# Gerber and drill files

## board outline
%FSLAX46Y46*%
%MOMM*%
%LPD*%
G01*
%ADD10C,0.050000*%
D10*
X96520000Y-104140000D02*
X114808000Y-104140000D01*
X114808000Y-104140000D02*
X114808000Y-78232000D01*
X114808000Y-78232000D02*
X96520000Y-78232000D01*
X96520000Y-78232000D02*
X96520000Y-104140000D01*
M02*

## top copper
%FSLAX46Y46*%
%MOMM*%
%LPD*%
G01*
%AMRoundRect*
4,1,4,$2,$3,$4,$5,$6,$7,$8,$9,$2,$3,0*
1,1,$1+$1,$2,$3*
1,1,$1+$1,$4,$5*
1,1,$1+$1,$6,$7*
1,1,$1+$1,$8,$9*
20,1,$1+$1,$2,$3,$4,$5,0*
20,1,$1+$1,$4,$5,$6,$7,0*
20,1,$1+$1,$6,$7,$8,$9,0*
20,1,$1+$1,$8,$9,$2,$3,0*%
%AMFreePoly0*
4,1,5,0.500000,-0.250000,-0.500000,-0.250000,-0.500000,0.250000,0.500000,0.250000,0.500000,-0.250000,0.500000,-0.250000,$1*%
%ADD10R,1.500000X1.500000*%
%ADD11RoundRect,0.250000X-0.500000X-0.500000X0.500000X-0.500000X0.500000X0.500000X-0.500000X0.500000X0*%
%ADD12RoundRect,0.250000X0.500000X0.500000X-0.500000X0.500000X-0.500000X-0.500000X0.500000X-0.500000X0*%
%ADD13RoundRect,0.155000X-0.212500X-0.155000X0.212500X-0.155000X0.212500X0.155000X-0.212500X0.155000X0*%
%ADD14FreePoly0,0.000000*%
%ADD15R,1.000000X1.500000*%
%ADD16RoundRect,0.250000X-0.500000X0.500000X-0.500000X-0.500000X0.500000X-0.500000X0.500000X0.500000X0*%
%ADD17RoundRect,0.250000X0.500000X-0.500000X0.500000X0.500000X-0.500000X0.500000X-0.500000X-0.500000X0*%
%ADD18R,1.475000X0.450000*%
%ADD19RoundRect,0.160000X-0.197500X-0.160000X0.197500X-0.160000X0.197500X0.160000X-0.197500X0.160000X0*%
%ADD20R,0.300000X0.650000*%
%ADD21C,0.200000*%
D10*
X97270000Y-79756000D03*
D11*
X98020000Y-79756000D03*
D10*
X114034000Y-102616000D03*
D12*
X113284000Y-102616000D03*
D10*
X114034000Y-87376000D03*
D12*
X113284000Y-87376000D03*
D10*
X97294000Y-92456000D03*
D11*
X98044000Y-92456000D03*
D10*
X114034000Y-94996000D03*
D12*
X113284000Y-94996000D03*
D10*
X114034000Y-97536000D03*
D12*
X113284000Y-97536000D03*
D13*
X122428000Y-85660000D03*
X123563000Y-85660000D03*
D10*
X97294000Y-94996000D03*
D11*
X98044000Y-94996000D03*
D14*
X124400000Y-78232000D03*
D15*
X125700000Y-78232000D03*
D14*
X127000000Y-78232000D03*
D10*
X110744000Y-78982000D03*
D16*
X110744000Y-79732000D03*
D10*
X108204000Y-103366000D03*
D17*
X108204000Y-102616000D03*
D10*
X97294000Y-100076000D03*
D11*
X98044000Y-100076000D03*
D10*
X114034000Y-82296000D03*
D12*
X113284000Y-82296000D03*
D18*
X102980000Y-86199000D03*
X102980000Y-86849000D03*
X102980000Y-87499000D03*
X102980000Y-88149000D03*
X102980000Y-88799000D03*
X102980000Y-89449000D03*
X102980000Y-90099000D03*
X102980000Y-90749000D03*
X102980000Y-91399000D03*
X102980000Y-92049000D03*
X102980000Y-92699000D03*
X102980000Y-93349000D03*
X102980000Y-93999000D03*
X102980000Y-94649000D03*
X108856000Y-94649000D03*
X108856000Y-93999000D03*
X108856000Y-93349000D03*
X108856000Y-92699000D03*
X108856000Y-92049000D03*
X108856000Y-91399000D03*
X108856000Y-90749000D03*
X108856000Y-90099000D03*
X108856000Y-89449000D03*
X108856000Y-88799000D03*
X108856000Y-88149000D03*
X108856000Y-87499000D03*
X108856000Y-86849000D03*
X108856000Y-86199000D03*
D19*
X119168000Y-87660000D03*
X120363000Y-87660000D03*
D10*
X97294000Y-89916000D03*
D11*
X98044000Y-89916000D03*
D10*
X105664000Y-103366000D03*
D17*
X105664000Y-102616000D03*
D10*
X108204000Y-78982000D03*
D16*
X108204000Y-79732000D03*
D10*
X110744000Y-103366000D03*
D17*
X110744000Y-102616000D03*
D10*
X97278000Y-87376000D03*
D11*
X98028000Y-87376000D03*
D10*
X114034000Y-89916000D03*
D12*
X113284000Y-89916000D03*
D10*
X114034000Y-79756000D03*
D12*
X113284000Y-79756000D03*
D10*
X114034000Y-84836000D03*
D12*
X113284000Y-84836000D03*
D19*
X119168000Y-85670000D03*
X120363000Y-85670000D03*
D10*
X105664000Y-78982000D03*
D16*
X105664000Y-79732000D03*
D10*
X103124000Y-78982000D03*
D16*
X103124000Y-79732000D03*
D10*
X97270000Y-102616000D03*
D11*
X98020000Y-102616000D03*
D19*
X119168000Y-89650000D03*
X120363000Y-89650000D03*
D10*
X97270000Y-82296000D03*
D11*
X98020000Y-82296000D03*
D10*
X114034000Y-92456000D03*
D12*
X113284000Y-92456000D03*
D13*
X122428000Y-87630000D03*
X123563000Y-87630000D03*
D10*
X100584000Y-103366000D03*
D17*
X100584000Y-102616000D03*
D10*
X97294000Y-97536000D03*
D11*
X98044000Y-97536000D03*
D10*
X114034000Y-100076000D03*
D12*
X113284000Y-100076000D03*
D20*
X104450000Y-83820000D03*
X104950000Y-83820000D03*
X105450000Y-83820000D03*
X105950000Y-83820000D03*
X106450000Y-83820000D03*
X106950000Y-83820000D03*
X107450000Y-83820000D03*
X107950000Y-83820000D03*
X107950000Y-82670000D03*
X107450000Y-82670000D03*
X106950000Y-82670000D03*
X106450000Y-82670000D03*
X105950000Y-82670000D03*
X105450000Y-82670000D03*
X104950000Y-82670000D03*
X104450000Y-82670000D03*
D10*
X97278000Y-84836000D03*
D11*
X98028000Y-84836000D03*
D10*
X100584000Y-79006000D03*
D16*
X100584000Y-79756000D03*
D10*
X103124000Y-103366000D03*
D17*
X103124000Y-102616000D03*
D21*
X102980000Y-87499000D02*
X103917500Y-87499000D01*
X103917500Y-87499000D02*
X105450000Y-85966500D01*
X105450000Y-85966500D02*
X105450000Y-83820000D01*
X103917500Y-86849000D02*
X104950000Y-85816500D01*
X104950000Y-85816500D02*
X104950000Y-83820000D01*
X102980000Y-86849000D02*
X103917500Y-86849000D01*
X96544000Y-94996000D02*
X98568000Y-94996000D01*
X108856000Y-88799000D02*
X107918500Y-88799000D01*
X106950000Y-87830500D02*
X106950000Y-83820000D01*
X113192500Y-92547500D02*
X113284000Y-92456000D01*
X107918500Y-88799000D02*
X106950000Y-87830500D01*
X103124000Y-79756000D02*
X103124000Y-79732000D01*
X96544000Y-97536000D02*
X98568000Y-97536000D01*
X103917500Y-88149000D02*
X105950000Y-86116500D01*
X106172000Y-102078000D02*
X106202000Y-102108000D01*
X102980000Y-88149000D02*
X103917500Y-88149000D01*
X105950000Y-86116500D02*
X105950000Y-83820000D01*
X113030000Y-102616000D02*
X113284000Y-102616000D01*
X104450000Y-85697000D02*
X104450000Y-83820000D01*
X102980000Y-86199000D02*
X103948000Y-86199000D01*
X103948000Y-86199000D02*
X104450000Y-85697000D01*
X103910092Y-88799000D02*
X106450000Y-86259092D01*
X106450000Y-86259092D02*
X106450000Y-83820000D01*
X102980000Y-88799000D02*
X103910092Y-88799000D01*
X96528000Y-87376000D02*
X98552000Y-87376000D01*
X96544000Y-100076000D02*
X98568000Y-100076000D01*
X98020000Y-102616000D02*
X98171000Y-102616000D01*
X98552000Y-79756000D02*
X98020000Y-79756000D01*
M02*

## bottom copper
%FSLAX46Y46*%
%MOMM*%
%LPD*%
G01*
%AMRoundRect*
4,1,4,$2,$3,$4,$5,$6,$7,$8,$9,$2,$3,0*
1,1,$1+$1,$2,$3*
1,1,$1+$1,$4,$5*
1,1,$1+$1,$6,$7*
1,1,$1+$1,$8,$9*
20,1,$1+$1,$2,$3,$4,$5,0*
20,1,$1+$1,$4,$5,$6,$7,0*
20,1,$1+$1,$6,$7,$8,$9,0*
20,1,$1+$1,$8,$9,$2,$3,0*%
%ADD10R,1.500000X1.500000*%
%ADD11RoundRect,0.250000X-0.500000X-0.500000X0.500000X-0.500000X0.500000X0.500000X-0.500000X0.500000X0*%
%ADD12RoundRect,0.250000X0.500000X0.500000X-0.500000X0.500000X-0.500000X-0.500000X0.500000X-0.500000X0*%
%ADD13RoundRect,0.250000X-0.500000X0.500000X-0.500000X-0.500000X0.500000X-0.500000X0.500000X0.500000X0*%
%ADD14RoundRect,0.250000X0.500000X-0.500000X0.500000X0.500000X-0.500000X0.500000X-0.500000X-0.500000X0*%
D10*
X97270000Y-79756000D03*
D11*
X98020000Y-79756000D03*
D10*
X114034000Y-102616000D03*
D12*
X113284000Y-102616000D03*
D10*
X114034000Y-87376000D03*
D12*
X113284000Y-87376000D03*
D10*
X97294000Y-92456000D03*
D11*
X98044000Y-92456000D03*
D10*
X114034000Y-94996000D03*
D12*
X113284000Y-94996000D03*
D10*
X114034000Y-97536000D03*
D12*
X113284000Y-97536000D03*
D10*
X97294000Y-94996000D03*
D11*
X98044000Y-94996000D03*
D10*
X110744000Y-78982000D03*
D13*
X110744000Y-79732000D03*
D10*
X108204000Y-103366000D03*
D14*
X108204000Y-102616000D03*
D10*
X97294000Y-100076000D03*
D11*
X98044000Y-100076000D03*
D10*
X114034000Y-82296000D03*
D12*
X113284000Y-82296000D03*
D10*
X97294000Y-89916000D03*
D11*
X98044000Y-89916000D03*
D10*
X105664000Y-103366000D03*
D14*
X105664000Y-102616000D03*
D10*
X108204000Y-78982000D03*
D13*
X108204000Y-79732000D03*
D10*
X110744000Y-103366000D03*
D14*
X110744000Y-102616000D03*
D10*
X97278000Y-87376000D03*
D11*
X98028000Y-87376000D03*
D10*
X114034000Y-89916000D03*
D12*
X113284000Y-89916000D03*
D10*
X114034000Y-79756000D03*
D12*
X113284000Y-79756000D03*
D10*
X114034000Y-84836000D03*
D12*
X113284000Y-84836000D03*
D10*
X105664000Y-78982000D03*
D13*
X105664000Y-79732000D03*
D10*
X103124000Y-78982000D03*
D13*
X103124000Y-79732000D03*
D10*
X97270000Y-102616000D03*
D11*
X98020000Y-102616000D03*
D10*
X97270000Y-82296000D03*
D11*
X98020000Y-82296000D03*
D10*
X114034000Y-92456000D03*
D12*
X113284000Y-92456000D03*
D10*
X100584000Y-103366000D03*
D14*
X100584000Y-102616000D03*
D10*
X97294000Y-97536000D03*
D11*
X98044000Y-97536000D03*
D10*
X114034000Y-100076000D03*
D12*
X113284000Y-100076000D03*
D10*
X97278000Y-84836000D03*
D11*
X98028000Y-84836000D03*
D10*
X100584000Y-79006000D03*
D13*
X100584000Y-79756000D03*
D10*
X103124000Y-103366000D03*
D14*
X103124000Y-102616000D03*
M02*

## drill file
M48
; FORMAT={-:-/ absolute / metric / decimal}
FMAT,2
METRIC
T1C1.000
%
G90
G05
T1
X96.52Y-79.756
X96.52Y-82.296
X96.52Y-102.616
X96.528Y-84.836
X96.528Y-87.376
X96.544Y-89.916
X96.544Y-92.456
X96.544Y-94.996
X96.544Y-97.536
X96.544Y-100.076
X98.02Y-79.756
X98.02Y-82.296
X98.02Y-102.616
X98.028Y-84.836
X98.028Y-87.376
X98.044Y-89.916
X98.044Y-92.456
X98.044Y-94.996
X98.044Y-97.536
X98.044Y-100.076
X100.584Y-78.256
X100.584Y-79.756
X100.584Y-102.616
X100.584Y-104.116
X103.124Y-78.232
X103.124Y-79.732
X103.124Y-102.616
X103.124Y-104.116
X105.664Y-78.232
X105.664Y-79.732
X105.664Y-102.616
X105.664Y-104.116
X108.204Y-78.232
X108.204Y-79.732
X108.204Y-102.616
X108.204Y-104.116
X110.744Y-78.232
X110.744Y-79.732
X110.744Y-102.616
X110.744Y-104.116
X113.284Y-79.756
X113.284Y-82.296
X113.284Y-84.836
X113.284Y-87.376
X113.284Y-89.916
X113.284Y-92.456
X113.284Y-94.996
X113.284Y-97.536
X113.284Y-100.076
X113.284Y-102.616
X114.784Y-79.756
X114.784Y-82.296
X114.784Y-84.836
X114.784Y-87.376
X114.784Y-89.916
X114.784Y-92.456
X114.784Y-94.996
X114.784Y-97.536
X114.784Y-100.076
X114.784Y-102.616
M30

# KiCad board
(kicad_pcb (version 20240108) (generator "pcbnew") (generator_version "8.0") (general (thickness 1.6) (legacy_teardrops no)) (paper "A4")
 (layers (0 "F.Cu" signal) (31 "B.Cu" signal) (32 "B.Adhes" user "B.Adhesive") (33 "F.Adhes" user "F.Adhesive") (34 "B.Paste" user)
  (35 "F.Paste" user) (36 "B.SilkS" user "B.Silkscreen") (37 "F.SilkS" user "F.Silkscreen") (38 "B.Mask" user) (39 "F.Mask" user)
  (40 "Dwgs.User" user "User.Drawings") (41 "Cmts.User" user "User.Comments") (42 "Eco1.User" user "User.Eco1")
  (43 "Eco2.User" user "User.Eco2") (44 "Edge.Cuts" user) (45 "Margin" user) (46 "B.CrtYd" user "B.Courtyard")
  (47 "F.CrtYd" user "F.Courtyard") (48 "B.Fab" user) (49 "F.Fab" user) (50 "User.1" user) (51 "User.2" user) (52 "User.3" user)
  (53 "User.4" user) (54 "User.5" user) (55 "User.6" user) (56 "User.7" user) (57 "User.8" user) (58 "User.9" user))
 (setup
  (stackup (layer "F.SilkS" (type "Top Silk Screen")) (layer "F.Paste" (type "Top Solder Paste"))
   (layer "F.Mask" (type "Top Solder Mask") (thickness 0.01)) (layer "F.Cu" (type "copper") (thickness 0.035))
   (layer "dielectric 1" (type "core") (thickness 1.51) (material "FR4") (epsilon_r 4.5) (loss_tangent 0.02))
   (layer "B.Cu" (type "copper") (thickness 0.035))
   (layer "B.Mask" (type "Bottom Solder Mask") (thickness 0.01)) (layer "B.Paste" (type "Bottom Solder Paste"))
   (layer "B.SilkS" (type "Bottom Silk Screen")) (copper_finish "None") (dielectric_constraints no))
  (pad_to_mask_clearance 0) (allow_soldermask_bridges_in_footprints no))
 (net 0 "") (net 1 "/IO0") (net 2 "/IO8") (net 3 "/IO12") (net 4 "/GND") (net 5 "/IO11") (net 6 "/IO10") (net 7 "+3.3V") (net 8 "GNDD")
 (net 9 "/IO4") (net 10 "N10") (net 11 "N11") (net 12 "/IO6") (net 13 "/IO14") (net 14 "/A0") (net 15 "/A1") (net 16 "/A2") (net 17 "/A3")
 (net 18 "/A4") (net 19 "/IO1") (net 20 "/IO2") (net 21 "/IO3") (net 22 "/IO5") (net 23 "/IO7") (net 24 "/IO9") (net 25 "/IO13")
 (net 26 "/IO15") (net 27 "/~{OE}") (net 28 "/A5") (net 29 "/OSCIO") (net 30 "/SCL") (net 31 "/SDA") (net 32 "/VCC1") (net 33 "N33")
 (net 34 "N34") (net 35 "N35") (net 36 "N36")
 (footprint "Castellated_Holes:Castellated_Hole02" (layer "F.Cu") (at 96.52 79.756)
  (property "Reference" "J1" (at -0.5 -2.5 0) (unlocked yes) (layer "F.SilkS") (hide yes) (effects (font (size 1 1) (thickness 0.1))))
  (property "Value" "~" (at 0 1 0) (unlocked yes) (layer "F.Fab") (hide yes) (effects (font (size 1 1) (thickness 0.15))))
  (pad "1" thru_hole rect (at 0 0) (size 1.5 1.5) (drill 1 (offset 0.75 0)) (layers "*.Cu" "*.Mask") (remove_unused_layers no)
   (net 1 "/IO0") (solder_mask_margin 0.04))
  (pad "1" thru_hole roundrect (at 1.5 0) (size 1.5 1.5) (drill 1) (layers "*.Cu" "*.Mask") (remove_unused_layers no)
   (roundrect_rratio 0.1666666667) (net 1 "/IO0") (solder_mask_margin 0.04)))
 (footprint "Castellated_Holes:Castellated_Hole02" (layer "F.Cu") (at 114.784 102.616 180)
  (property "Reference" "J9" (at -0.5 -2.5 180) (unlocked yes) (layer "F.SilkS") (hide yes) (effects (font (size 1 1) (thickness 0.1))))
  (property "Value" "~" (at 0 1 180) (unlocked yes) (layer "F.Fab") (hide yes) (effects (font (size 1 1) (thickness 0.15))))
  (pad "1" thru_hole rect (at 0 0 180) (size 1.5 1.5) (drill 1 (offset 0.75 0)) (layers "*.Cu" "*.Mask") (remove_unused_layers no)
   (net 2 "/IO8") (solder_mask_margin 0.04))
  (pad "1" thru_hole roundrect (at 1.5 0 180) (size 1.5 1.5) (drill 1) (layers "*.Cu" "*.Mask") (remove_unused_layers no)
   (roundrect_rratio 0.1666666667) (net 2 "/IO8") (solder_mask_margin 0.04)))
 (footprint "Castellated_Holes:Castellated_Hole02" (layer "F.Cu") (at 114.784 87.376 180)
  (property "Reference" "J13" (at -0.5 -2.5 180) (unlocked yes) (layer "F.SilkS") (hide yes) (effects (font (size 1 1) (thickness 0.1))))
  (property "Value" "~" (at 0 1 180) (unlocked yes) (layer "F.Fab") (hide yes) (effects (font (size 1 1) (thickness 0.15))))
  (pad "1" thru_hole rect (at 0 0 180) (size 1.5 1.5) (drill 1 (offset 0.75 0)) (layers "*.Cu" "*.Mask") (remove_unused_layers no)
   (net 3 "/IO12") (solder_mask_margin 0.04))
  (pad "1" thru_hole roundrect (at 1.5 0 180) (size 1.5 1.5) (drill 1) (layers "*.Cu" "*.Mask") (remove_unused_layers no)
   (roundrect_rratio 0.1666666667) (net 3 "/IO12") (solder_mask_margin 0.04)))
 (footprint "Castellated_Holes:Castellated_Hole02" (layer "F.Cu") (at 96.544 92.456)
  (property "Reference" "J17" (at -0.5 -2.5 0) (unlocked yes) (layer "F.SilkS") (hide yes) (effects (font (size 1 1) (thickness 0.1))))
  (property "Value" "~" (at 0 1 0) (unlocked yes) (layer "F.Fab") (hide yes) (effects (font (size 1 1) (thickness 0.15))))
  (pad "1" thru_hole rect (at 0 0) (size 1.5 1.5) (drill 1 (offset 0.75 0)) (layers "*.Cu" "*.Mask") (remove_unused_layers no)
   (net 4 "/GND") (solder_mask_margin 0.04))
  (pad "1" thru_hole roundrect (at 1.5 0) (size 1.5 1.5) (drill 1) (layers "*.Cu" "*.Mask") (remove_unused_layers no)
   (roundrect_rratio 0.1666666667) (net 4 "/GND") (solder_mask_margin 0.04)))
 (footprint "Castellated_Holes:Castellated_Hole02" (layer "F.Cu") (at 114.784 94.996 180)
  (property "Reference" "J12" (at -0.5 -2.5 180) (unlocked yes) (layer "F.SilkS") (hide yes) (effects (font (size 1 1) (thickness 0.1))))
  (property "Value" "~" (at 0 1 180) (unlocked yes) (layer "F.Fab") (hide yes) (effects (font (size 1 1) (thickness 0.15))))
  (pad "1" thru_hole rect (at 0 0 180) (size 1.5 1.5) (drill 1 (offset 0.75 0)) (layers "*.Cu" "*.Mask") (remove_unused_layers no)
   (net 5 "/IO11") (solder_mask_margin 0.04))
  (pad "1" thru_hole roundrect (at 1.5 0 180) (size 1.5 1.5) (drill 1) (layers "*.Cu" "*.Mask") (remove_unused_layers no)
   (roundrect_rratio 0.1666666667) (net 5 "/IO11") (solder_mask_margin 0.04)))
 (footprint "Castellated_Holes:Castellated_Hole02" (layer "F.Cu") (at 114.784 97.536 180)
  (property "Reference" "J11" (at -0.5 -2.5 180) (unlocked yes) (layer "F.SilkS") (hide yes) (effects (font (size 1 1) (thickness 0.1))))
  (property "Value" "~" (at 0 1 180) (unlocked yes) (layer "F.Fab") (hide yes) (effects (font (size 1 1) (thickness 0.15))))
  (pad "1" thru_hole rect (at 0 0 180) (size 1.5 1.5) (drill 1 (offset 0.75 0)) (layers "*.Cu" "*.Mask") (remove_unused_layers no)
   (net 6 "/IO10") (solder_mask_margin 0.04))
  (pad "1" thru_hole roundrect (at 1.5 0 180) (size 1.5 1.5) (drill 1) (layers "*.Cu" "*.Mask") (remove_unused_layers no)
   (roundrect_rratio 0.1666666667) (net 6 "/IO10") (solder_mask_margin 0.04)))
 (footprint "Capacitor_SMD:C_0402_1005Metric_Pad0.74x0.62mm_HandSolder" (layer "F.Cu") (at 122.9955 85.66)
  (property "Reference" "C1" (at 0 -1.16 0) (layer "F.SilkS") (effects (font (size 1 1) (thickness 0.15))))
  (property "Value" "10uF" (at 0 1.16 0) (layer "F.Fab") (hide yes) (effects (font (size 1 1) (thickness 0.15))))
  (pad "1" smd roundrect (at -0.5675 0) (size 0.735 0.62) (layers "F.Cu" "F.Paste" "F.Mask") (roundrect_rratio 0.25) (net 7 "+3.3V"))
  (pad "2" smd roundrect (at 0.5675 0) (size 0.735 0.62) (layers "F.Cu" "F.Paste" "F.Mask") (roundrect_rratio 0.25) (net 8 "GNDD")))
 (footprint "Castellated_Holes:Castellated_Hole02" (layer "F.Cu") (at 96.544 94.996)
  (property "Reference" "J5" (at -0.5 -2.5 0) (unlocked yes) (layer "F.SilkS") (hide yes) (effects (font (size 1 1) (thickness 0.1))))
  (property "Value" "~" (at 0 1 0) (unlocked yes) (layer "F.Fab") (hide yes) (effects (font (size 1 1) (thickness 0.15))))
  (pad "1" thru_hole rect (at 0 0) (size 1.5 1.5) (drill 1 (offset 0.75 0)) (layers "*.Cu" "*.Mask") (remove_unused_layers no)
   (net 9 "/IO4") (solder_mask_margin 0.04))
  (pad "1" thru_hole roundrect (at 1.5 0) (size 1.5 1.5) (drill 1) (layers "*.Cu" "*.Mask") (remove_unused_layers no)
   (roundrect_rratio 0.1666666667) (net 9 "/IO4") (solder_mask_margin 0.04)))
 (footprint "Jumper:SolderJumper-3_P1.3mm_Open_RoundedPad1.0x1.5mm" (layer "F.Cu") (at 125.7 78.232)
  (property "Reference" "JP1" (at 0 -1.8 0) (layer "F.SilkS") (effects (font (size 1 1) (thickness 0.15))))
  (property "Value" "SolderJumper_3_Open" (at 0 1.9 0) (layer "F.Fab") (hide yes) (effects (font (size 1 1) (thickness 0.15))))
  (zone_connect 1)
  (pad "1" smd custom (at -1.3 0) (size 1 0.5) (layers "F.Cu" "F.Mask") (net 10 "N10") (zone_connect 2) (thermal_bridge_angle 45)
   (options (clearance outline) (anchor rect)) (primitives))
  (pad "2" smd rect (at 0 0) (size 1 1.5) (layers "F.Cu" "F.Mask") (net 7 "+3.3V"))
  (pad "3" smd custom (at 1.3 0) (size 1 0.5) (layers "F.Cu" "F.Mask") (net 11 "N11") (zone_connect 2) (thermal_bridge_angle 45)
   (options (clearance outline) (anchor rect)) (primitives)))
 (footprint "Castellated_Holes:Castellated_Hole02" (layer "F.Cu") (at 110.744 78.232 -90)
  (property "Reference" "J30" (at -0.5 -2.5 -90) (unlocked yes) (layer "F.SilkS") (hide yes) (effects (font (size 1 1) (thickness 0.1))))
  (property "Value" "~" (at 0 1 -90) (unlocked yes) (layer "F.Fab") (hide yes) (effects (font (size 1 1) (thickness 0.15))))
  (pad "1" thru_hole rect (at 0 0 270) (size 1.5 1.5) (drill 1 (offset 0.75 0)) (layers "*.Cu" "*.Mask") (remove_unused_layers no)
   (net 8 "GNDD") (solder_mask_margin 0.04))
  (pad "1" thru_hole roundrect (at 1.5 0 270) (size 1.5 1.5) (drill 1) (layers "*.Cu" "*.Mask") (remove_unused_layers no)
   (roundrect_rratio 0.1666666667) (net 8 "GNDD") (solder_mask_margin 0.04)))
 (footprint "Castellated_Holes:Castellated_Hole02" (layer "F.Cu") (at 108.204 104.116 90)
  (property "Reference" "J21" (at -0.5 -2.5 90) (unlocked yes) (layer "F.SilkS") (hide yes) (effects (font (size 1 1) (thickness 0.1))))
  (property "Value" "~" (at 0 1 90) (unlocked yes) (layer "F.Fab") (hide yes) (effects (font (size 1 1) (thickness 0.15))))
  (pad "1" thru_hole rect (at 0 0 90) (size 1.5 1.5) (drill 1 (offset 0.75 0)) (layers "*.Cu" "*.Mask") (remove_unused_layers no)
   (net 7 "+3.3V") (solder_mask_margin 0.04))
  (pad "1" thru_hole roundrect (at 1.5 0 90) (size 1.5 1.5) (drill 1) (layers "*.Cu" "*.Mask") (remove_unused_layers no)
   (roundrect_rratio 0.1666666667) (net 7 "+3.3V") (solder_mask_margin 0.04)))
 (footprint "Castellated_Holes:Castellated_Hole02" (layer "F.Cu") (at 96.544 100.076)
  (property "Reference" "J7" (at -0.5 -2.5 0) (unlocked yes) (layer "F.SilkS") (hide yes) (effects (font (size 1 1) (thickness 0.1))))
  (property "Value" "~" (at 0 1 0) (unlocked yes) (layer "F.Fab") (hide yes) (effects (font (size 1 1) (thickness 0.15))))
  (pad "1" thru_hole rect (at 0 0) (size 1.5 1.5) (drill 1 (offset 0.75 0)) (layers "*.Cu" "*.Mask") (remove_unused_layers no)
   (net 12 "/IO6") (solder_mask_margin 0.04))
  (pad "1" thru_hole roundrect (at 1.5 0) (size 1.5 1.5) (drill 1) (layers "*.Cu" "*.Mask") (remove_unused_layers no)
   (roundrect_rratio 0.1666666667) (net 12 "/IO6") (solder_mask_margin 0.04)))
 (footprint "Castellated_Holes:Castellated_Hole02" (layer "F.Cu") (at 114.784 82.296 180)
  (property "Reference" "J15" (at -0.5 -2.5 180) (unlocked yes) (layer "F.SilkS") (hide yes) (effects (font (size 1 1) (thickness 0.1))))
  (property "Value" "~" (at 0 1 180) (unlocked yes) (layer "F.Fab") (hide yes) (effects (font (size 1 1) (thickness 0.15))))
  (pad "1" thru_hole rect (at 0 0 180) (size 1.5 1.5) (drill 1 (offset 0.75 0)) (layers "*.Cu" "*.Mask") (remove_unused_layers no)
   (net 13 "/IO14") (solder_mask_margin 0.04))
  (pad "1" thru_hole roundrect (at 1.5 0 180) (size 1.5 1.5) (drill 1) (layers "*.Cu" "*.Mask") (remove_unused_layers no)
   (roundrect_rratio 0.1666666667) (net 13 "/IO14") (solder_mask_margin 0.04)))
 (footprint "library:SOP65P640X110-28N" (layer "F.Cu") (at 105.918 90.424)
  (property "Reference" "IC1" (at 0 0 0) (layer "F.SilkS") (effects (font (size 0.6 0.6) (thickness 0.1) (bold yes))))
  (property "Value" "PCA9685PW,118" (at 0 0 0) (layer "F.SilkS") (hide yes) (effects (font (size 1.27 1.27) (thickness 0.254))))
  (pad "1" smd rect (at -2.938 -4.225 90) (size 0.45 1.475) (layers "F.Cu" "F.Paste" "F.Mask") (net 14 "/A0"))
  (pad "2" smd rect (at -2.938 -3.575 90) (size 0.45 1.475) (layers "F.Cu" "F.Paste" "F.Mask") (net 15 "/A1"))
  (pad "3" smd rect (at -2.938 -2.925 90) (size 0.45 1.475) (layers "F.Cu" "F.Paste" "F.Mask") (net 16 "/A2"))
  (pad "4" smd rect (at -2.938 -2.275 90) (size 0.45 1.475) (layers "F.Cu" "F.Paste" "F.Mask") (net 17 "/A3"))
  (pad "5" smd rect (at -2.938 -1.625 90) (size 0.45 1.475) (layers "F.Cu" "F.Paste" "F.Mask") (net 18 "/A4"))
  (pad "6" smd rect (at -2.938 -0.975 90) (size 0.45 1.475) (layers "F.Cu" "F.Paste" "F.Mask") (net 1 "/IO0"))
  (pad "7" smd rect (at -2.938 -0.325 90) (size 0.45 1.475) (layers "F.Cu" "F.Paste" "F.Mask") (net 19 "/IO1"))
  (pad "8" smd rect (at -2.938 0.325 90) (size 0.45 1.475) (layers "F.Cu" "F.Paste" "F.Mask") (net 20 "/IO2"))
  (pad "9" smd rect (at -2.938 0.975 90) (size 0.45 1.475) (layers "F.Cu" "F.Paste" "F.Mask") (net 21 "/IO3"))
  (pad "10" smd rect (at -2.938 1.625 90) (size 0.45 1.475) (layers "F.Cu" "F.Paste" "F.Mask") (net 9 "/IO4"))
  (pad "11" smd rect (at -2.938 2.275 90) (size 0.45 1.475) (layers "F.Cu" "F.Paste" "F.Mask") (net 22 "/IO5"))
  (pad "12" smd rect (at -2.938 2.925 90) (size 0.45 1.475) (layers "F.Cu" "F.Paste" "F.Mask") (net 12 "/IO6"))
  (pad "13" smd rect (at -2.938 3.575 90) (size 0.45 1.475) (layers "F.Cu" "F.Paste" "F.Mask") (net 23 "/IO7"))
  (pad "14" smd rect (at -2.938 4.225 90) (size 0.45 1.475) (layers "F.Cu" "F.Paste" "F.Mask") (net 8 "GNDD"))
  (pad "15" smd rect (at 2.938 4.225 90) (size 0.45 1.475) (layers "F.Cu" "F.Paste" "F.Mask") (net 2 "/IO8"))
  (pad "16" smd rect (at 2.938 3.575 90) (size 0.45 1.475) (layers "F.Cu" "F.Paste" "F.Mask") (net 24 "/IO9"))
  (pad "17" smd rect (at 2.938 2.925 90) (size 0.45 1.475) (layers "F.Cu" "F.Paste" "F.Mask") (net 6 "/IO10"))
  (pad "18" smd rect (at 2.938 2.275 90) (size 0.45 1.475) (layers "F.Cu" "F.Paste" "F.Mask") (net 5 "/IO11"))
  (pad "19" smd rect (at 2.938 1.625 90) (size 0.45 1.475) (layers "F.Cu" "F.Paste" "F.Mask") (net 3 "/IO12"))
  (pad "20" smd rect (at 2.938 0.975 90) (size 0.45 1.475) (layers "F.Cu" "F.Paste" "F.Mask") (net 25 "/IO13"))
  (pad "21" smd rect (at 2.938 0.325 90) (size 0.45 1.475) (layers "F.Cu" "F.Paste" "F.Mask") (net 13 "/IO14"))
  (pad "22" smd rect (at 2.938 -0.325 90) (size 0.45 1.475) (layers "F.Cu" "F.Paste" "F.Mask") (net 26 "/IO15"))
  (pad "23" smd rect (at 2.938 -0.975 90) (size 0.45 1.475) (layers "F.Cu" "F.Paste" "F.Mask") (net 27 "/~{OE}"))
  (pad "24" smd rect (at 2.938 -1.625 90) (size 0.45 1.475) (layers "F.Cu" "F.Paste" "F.Mask") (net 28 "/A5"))
  (pad "25" smd rect (at 2.938 -2.275 90) (size 0.45 1.475) (layers "F.Cu" "F.Paste" "F.Mask") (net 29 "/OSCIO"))
  (pad "26" smd rect (at 2.938 -2.925 90) (size 0.45 1.475) (layers "F.Cu" "F.Paste" "F.Mask") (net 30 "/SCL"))
  (pad "27" smd rect (at 2.938 -3.575 90) (size 0.45 1.475) (layers "F.Cu" "F.Paste" "F.Mask") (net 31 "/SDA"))
  (pad "28" smd rect (at 2.938 -4.225 90) (size 0.45 1.475) (layers "F.Cu" "F.Paste" "F.Mask") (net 7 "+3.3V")))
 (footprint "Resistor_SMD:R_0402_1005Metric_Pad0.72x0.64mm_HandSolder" (layer "F.Cu") (at 119.7655 87.66)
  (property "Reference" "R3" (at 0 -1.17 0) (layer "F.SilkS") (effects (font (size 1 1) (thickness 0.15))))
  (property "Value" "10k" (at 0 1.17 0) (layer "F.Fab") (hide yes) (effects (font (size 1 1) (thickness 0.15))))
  (pad "1" smd roundrect (at -0.5975 0) (size 0.715 0.64) (layers "F.Cu" "F.Paste" "F.Mask") (roundrect_rratio 0.25) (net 30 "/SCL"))
  (pad "2" smd roundrect (at 0.5975 0) (size 0.715 0.64) (layers "F.Cu" "F.Paste" "F.Mask") (roundrect_rratio 0.25) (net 11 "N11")))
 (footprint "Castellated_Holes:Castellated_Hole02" (layer "F.Cu") (at 96.544 89.916)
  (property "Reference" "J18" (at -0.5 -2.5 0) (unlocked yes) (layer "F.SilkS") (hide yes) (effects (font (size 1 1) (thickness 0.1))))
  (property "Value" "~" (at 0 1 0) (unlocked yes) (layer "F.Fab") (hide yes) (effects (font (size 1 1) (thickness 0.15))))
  (pad "1" thru_hole rect (at 0 0) (size 1.5 1.5) (drill 1 (offset 0.75 0)) (layers "*.Cu" "*.Mask") (remove_unused_layers no)
   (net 8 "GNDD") (solder_mask_margin 0.04))
  (pad "1" thru_hole roundrect (at 1.5 0) (size 1.5 1.5) (drill 1) (layers "*.Cu" "*.Mask") (remove_unused_layers no)
   (roundrect_rratio 0.1666666667) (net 8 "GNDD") (solder_mask_margin 0.04)))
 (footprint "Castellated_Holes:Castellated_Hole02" (layer "F.Cu") (at 105.664 104.116 90)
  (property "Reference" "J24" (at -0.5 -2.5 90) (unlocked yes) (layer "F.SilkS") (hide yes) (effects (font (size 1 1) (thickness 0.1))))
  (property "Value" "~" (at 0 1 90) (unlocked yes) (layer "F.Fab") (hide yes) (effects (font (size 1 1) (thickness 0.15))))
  (pad "1" thru_hole rect (at 0 0 90) (size 1.5 1.5) (drill 1 (offset 0.75 0)) (layers "*.Cu" "*.Mask") (remove_unused_layers no)
   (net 17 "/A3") (solder_mask_margin 0.04))
  (pad "1" thru_hole roundrect (at 1.5 0 90) (size 1.5 1.5) (drill 1) (layers "*.Cu" "*.Mask") (remove_unused_layers no)
   (roundrect_rratio 0.1666666667) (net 17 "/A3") (solder_mask_margin 0.04)))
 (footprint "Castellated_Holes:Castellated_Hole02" (layer "F.Cu") (at 108.204 78.232 -90)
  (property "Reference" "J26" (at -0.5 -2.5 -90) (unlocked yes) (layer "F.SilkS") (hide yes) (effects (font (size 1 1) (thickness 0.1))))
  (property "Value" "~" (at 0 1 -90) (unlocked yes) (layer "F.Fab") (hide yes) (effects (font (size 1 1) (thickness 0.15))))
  (pad "1" thru_hole rect (at 0 0 270) (size 1.5 1.5) (drill 1 (offset 0.75 0)) (layers "*.Cu" "*.Mask") (remove_unused_layers no)
   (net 15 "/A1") (solder_mask_margin 0.04))
  (pad "1" thru_hole roundrect (at 1.5 0 270) (size 1.5 1.5) (drill 1) (layers "*.Cu" "*.Mask") (remove_unused_layers no)
   (roundrect_rratio 0.1666666667) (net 15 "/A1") (solder_mask_margin 0.04)))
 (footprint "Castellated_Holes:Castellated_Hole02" (layer "F.Cu") (at 110.744 104.116 90)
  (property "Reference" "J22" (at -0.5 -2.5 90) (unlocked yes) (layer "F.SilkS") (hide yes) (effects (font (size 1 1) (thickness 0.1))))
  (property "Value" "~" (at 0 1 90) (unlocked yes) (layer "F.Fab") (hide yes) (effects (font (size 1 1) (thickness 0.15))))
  (pad "1" thru_hole rect (at 0 0 90) (size 1.5 1.5) (drill 1 (offset 0.75 0)) (layers "*.Cu" "*.Mask") (remove_unused_layers no)
   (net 8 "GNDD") (solder_mask_margin 0.04))
  (pad "1" thru_hole roundrect (at 1.5 0 90) (size 1.5 1.5) (drill 1) (layers "*.Cu" "*.Mask") (remove_unused_layers no)
   (roundrect_rratio 0.1666666667) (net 8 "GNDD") (solder_mask_margin 0.04)))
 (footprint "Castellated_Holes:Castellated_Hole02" (layer "F.Cu") (at 96.528 87.376)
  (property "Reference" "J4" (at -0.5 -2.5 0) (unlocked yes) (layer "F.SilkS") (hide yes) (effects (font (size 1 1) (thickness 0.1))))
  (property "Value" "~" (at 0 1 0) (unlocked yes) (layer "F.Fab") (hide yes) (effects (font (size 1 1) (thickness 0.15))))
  (pad "1" thru_hole rect (at 0 0) (size 1.5 1.5) (drill 1 (offset 0.75 0)) (layers "*.Cu" "*.Mask") (remove_unused_layers no)
   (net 21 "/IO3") (solder_mask_margin 0.04))
  (pad "1" thru_hole roundrect (at 1.5 0) (size 1.5 1.5) (drill 1) (layers "*.Cu" "*.Mask") (remove_unused_layers no)
   (roundrect_rratio 0.1666666667) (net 21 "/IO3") (solder_mask_margin 0.04)))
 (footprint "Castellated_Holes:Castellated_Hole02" (layer "F.Cu") (at 114.784 89.916 180)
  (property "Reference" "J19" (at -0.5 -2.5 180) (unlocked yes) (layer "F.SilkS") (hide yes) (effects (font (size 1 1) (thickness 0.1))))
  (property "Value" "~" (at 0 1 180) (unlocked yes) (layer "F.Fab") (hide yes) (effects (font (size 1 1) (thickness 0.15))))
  (pad "1" thru_hole rect (at 0 0 180) (size 1.5 1.5) (drill 1 (offset 0.75 0)) (layers "*.Cu" "*.Mask") (remove_unused_layers no)
   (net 18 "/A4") (solder_mask_margin 0.04))
  (pad "1" thru_hole roundrect (at 1.5 0 180) (size 1.5 1.5) (drill 1) (layers "*.Cu" "*.Mask") (remove_unused_layers no)
   (roundrect_rratio 0.1666666667) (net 18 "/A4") (solder_mask_margin 0.04)))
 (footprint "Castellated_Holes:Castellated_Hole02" (layer "F.Cu") (at 114.784 79.756 180)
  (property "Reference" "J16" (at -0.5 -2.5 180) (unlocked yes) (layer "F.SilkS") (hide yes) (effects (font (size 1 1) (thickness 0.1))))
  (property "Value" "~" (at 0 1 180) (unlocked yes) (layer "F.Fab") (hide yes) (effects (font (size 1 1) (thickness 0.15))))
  (pad "1" thru_hole rect (at 0 0 180) (size 1.5 1.5) (drill 1 (offset 0.75 0)) (layers "*.Cu" "*.Mask") (remove_unused_layers no)
   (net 26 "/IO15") (solder_mask_margin 0.04))
  (pad "1" thru_hole roundrect (at 1.5 0 180) (size 1.5 1.5) (drill 1) (layers "*.Cu" "*.Mask") (remove_unused_layers no)
   (roundrect_rratio 0.1666666667) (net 26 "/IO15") (solder_mask_margin 0.04)))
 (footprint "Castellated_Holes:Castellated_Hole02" (layer "F.Cu") (at 114.784 84.836 180)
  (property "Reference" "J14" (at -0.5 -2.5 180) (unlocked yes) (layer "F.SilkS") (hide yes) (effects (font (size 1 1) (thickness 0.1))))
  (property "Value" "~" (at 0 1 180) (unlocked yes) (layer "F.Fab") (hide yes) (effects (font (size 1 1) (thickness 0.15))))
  (pad "1" thru_hole rect (at 0 0 180) (size 1.5 1.5) (drill 1 (offset 0.75 0)) (layers "*.Cu" "*.Mask") (remove_unused_layers no)
   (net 25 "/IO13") (solder_mask_margin 0.04))
  (pad "1" thru_hole roundrect (at 1.5 0 180) (size 1.5 1.5) (drill 1) (layers "*.Cu" "*.Mask") (remove_unused_layers no)
   (roundrect_rratio 0.1666666667) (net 25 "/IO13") (solder_mask_margin 0.04)))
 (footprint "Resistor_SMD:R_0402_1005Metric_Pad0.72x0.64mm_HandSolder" (layer "F.Cu") (at 119.7655 85.67)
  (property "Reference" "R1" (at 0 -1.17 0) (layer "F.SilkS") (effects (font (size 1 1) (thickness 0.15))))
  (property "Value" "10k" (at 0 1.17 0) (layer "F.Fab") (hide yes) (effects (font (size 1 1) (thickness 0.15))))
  (pad "1" smd roundrect (at -0.5975 0) (size 0.715 0.64) (layers "F.Cu" "F.Paste" "F.Mask") (roundrect_rratio 0.25) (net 8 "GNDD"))
  (pad "2" smd roundrect (at 0.5975 0) (size 0.715 0.64) (layers "F.Cu" "F.Paste" "F.Mask") (roundrect_rratio 0.25) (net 27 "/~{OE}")))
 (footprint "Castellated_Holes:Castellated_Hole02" (layer "F.Cu") (at 105.664 78.232 -90)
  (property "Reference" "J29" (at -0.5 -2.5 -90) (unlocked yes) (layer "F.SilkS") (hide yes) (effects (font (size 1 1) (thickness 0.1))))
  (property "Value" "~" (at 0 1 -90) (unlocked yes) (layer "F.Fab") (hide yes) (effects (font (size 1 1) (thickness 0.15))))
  (pad "1" thru_hole rect (at 0 0 270) (size 1.5 1.5) (drill 1 (offset 0.75 0)) (layers "*.Cu" "*.Mask") (remove_unused_layers no)
   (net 31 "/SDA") (solder_mask_margin 0.04))
  (pad "1" thru_hole roundrect (at 1.5 0 270) (size 1.5 1.5) (drill 1) (layers "*.Cu" "*.Mask") (remove_unused_layers no)
   (roundrect_rratio 0.1666666667) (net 31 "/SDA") (solder_mask_margin 0.04)))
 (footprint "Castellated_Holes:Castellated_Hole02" (layer "F.Cu") (at 103.124 78.232 -90)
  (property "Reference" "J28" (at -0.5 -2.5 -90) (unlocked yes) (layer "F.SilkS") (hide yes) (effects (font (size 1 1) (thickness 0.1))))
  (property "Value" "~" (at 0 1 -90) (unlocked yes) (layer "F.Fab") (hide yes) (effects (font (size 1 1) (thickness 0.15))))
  (pad "1" thru_hole rect (at 0 0 270) (size 1.5 1.5) (drill 1 (offset 0.75 0)) (layers "*.Cu" "*.Mask") (remove_unused_layers no)
   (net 30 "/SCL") (solder_mask_margin 0.04))
  (pad "1" thru_hole roundrect (at 1.5 0 270) (size 1.5 1.5) (drill 1) (layers "*.Cu" "*.Mask") (remove_unused_layers no)
   (roundrect_rratio 0.1666666667) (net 30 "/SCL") (solder_mask_margin 0.04)))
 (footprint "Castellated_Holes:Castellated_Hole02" (layer "F.Cu") (at 96.52 102.616)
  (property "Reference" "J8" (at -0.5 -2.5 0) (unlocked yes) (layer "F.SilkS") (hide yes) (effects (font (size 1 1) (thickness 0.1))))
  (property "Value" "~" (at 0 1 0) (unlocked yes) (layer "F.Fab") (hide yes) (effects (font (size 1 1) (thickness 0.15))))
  (pad "1" thru_hole rect (at 0 0) (size 1.5 1.5) (drill 1 (offset 0.75 0)) (layers "*.Cu" "*.Mask") (remove_unused_layers no)
   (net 23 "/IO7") (solder_mask_margin 0.04))
  (pad "1" thru_hole roundrect (at 1.5 0) (size 1.5 1.5) (drill 1) (layers "*.Cu" "*.Mask") (remove_unused_layers no)
   (roundrect_rratio 0.1666666667) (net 23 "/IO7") (solder_mask_margin 0.04)))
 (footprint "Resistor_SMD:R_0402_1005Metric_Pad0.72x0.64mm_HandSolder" (layer "F.Cu") (at 119.7655 89.65)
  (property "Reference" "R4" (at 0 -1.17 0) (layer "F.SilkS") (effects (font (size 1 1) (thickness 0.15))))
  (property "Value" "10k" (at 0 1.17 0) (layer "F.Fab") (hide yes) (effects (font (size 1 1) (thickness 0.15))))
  (pad "1" smd roundrect (at -0.5975 0) (size 0.715 0.64) (layers "F.Cu" "F.Paste" "F.Mask") (roundrect_rratio 0.25) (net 31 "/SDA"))
  (pad "2" smd roundrect (at 0.5975 0) (size 0.715 0.64) (layers "F.Cu" "F.Paste" "F.Mask") (roundrect_rratio 0.25) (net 10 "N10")))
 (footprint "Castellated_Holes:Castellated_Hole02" (layer "F.Cu") (at 96.52 82.296)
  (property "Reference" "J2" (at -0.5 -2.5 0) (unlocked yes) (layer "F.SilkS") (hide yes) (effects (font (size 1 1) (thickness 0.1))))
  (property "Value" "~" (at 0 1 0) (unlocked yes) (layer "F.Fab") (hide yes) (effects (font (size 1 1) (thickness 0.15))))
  (pad "1" thru_hole rect (at 0 0) (size 1.5 1.5) (drill 1 (offset 0.75 0)) (layers "*.Cu" "*.Mask") (remove_unused_layers no)
   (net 19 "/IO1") (solder_mask_margin 0.04))
  (pad "1" thru_hole roundrect (at 1.5 0) (size 1.5 1.5) (drill 1) (layers "*.Cu" "*.Mask") (remove_unused_layers no)
   (roundrect_rratio 0.1666666667) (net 19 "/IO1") (solder_mask_margin 0.04)))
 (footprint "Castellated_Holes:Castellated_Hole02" (layer "F.Cu") (at 114.784 92.456 180)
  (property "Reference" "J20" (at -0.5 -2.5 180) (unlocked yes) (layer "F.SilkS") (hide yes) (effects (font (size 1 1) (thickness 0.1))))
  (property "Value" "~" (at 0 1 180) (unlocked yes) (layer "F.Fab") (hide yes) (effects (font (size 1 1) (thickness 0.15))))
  (pad "1" thru_hole rect (at 0 0 180) (size 1.5 1.5) (drill 1 (offset 0.75 0)) (layers "*.Cu" "*.Mask") (remove_unused_layers no)
   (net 28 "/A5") (solder_mask_margin 0.04))
  (pad "1" thru_hole roundrect (at 1.5 0 180) (size 1.5 1.5) (drill 1) (layers "*.Cu" "*.Mask") (remove_unused_layers no)
   (roundrect_rratio 0.1666666667) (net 28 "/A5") (solder_mask_margin 0.04)))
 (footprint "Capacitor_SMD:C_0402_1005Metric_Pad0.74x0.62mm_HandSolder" (layer "F.Cu") (at 122.9955 87.63)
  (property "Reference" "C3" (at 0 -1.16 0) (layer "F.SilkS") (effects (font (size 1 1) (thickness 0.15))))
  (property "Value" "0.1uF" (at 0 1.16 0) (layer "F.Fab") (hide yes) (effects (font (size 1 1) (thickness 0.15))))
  (pad "1" smd roundrect (at -0.5675 0) (size 0.735 0.62) (layers "F.Cu" "F.Paste" "F.Mask") (roundrect_rratio 0.25) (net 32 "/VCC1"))
  (pad "2" smd roundrect (at 0.5675 0) (size 0.735 0.62) (layers "F.Cu" "F.Paste" "F.Mask") (roundrect_rratio 0.25) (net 8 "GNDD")))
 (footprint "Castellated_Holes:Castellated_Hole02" (layer "F.Cu") (at 100.584 104.116 90)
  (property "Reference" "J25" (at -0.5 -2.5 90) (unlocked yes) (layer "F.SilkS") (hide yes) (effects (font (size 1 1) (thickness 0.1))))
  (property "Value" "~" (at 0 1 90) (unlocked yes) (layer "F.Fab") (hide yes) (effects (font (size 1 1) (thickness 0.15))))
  (pad "1" thru_hole rect (at 0 0 90) (size 1.5 1.5) (drill 1 (offset 0.75 0)) (layers "*.Cu" "*.Mask") (remove_unused_layers no)
   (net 14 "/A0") (solder_mask_margin 0.04))
  (pad "1" thru_hole roundrect (at 1.5 0 90) (size 1.5 1.5) (drill 1) (layers "*.Cu" "*.Mask") (remove_unused_layers no)
   (roundrect_rratio 0.1666666667) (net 14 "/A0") (solder_mask_margin 0.04)))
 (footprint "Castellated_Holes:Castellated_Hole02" (layer "F.Cu") (at 96.544 97.536)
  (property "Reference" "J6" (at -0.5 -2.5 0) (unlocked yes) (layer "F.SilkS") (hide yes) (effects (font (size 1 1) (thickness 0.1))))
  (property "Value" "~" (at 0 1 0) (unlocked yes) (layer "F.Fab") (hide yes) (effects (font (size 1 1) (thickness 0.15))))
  (pad "1" thru_hole rect (at 0 0) (size 1.5 1.5) (drill 1 (offset 0.75 0)) (layers "*.Cu" "*.Mask") (remove_unused_layers no)
   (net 22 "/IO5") (solder_mask_margin 0.04))
  (pad "1" thru_hole roundrect (at 1.5 0) (size 1.5 1.5) (drill 1) (layers "*.Cu" "*.Mask") (remove_unused_layers no)
   (roundrect_rratio 0.1666666667) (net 22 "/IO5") (solder_mask_margin 0.04)))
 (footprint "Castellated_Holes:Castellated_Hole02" (layer "F.Cu") (at 114.784 100.076 180)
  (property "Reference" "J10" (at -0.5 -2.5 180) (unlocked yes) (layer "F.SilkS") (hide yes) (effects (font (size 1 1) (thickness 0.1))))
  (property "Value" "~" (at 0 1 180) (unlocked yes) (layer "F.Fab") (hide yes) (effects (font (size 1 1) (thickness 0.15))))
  (pad "1" thru_hole rect (at 0 0 180) (size 1.5 1.5) (drill 1 (offset 0.75 0)) (layers "*.Cu" "*.Mask") (remove_unused_layers no)
   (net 24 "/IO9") (solder_mask_margin 0.04))
  (pad "1" thru_hole roundrect (at 1.5 0 180) (size 1.5 1.5) (drill 1) (layers "*.Cu" "*.Mask") (remove_unused_layers no)
   (roundrect_rratio 0.1666666667) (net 24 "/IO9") (solder_mask_margin 0.04)))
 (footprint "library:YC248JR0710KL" (layer "F.Cu") (at 106.2 83.245)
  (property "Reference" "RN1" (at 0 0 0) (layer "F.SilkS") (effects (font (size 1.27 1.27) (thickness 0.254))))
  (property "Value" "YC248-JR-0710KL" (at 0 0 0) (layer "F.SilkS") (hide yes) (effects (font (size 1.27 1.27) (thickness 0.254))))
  (pad "1" smd rect (at -1.75 0.575) (size 0.3 0.65) (layers "F.Cu" "F.Paste" "F.Mask") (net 14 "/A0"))
  (pad "2" smd rect (at -1.25 0.575) (size 0.3 0.65) (layers "F.Cu" "F.Paste" "F.Mask") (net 15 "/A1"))
  (pad "3" smd rect (at -0.75 0.575) (size 0.3 0.65) (layers "F.Cu" "F.Paste" "F.Mask") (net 16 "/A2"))
  (pad "4" smd rect (at -0.25 0.575) (size 0.3 0.65) (layers "F.Cu" "F.Paste" "F.Mask") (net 17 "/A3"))
  (pad "5" smd rect (at 0.25 0.575) (size 0.3 0.65) (layers "F.Cu" "F.Paste" "F.Mask") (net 18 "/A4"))
  (pad "6" smd rect (at 0.75 0.575) (size 0.3 0.65) (layers "F.Cu" "F.Paste" "F.Mask") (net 28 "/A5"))
  (pad "7" smd rect (at 1.25 0.575) (size 0.3 0.65) (layers "F.Cu" "F.Paste" "F.Mask") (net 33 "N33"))
  (pad "8" smd rect (at 1.75 0.575) (size 0.3 0.65) (layers "F.Cu" "F.Paste" "F.Mask") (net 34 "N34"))
  (pad "9" smd rect (at 1.75 -0.575) (size 0.3 0.65) (layers "F.Cu" "F.Paste" "F.Mask") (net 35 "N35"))
  (pad "10" smd rect (at 1.25 -0.575) (size 0.3 0.65) (layers "F.Cu" "F.Paste" "F.Mask") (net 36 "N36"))
  (pad "11" smd rect (at 0.75 -0.575) (size 0.3 0.65) (layers "F.Cu" "F.Paste" "F.Mask") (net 8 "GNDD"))
  (pad "12" smd rect (at 0.25 -0.575) (size 0.3 0.65) (layers "F.Cu" "F.Paste" "F.Mask") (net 8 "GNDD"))
  (pad "13" smd rect (at -0.25 -0.575) (size 0.3 0.65) (layers "F.Cu" "F.Paste" "F.Mask") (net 8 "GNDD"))
  (pad "14" smd rect (at -0.75 -0.575) (size 0.3 0.65) (layers "F.Cu" "F.Paste" "F.Mask") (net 8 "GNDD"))
  (pad "15" smd rect (at -1.25 -0.575) (size 0.3 0.65) (layers "F.Cu" "F.Paste" "F.Mask") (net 8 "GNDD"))
  (pad "16" smd rect (at -1.75 -0.575) (size 0.3 0.65) (layers "F.Cu" "F.Paste" "F.Mask") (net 8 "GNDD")))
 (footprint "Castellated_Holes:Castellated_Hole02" (layer "F.Cu") (at 96.528 84.836)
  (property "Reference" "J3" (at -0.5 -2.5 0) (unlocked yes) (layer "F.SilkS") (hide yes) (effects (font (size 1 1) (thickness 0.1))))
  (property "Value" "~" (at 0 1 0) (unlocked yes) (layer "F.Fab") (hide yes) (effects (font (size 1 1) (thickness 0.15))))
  (pad "1" thru_hole rect (at 0 0) (size 1.5 1.5) (drill 1 (offset 0.75 0)) (layers "*.Cu" "*.Mask") (remove_unused_layers no)
   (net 20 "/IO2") (solder_mask_margin 0.04))
  (pad "1" thru_hole roundrect (at 1.5 0) (size 1.5 1.5) (drill 1) (layers "*.Cu" "*.Mask") (remove_unused_layers no)
   (roundrect_rratio 0.1666666667) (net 20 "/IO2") (solder_mask_margin 0.04)))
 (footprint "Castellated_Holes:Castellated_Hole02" (layer "F.Cu") (at 100.584 78.256 -90)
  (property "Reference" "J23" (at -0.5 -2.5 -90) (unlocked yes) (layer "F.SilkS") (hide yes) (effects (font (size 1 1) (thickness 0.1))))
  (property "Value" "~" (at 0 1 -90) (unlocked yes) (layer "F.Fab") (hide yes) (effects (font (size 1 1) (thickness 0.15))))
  (pad "1" thru_hole rect (at 0 0 270) (size 1.5 1.5) (drill 1 (offset 0.75 0)) (layers "*.Cu" "*.Mask") (remove_unused_layers no)
   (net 16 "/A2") (solder_mask_margin 0.04))
  (pad "1" thru_hole roundrect (at 1.5 0 270) (size 1.5 1.5) (drill 1) (layers "*.Cu" "*.Mask") (remove_unused_layers no)
   (roundrect_rratio 0.1666666667) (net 16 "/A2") (solder_mask_margin 0.04)))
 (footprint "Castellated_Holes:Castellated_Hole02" (layer "F.Cu") (at 103.124 104.116 90)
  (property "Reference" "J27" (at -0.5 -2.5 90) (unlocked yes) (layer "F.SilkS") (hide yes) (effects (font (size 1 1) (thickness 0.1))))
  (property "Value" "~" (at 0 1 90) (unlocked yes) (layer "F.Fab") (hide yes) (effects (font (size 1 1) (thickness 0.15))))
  (pad "1" thru_hole rect (at 0 0 90) (size 1.5 1.5) (drill 1 (offset 0.75 0)) (layers "*.Cu" "*.Mask") (remove_unused_layers no)
   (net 29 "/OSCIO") (solder_mask_margin 0.04))
  (pad "1" thru_hole roundrect (at 1.5 0 90) (size 1.5 1.5) (drill 1) (layers "*.Cu" "*.Mask") (remove_unused_layers no)
   (roundrect_rratio 0.1666666667) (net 29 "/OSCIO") (solder_mask_margin 0.04)))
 (gr_line (start 96.52 104.14) (end 114.808 104.14) (stroke (width 0.05) (type default)) (layer "Edge.Cuts"))
 (gr_line (start 114.808 104.14) (end 114.808 78.232) (stroke (width 0.05) (type default)) (layer "Edge.Cuts"))
 (gr_line (start 114.808 78.232) (end 96.52 78.232) (stroke (width 0.05) (type default)) (layer "Edge.Cuts"))
 (gr_line (start 96.52 78.232) (end 96.52 104.14) (stroke (width 0.05) (type default)) (layer "Edge.Cuts"))
 (segment (start 102.98 87.499) (end 103.9175 87.499) (width 0.2) (layer "F.Cu") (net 16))
 (segment (start 103.9175 87.499) (end 105.45 85.9665) (width 0.2) (layer "F.Cu") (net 16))
 (segment (start 105.45 85.9665) (end 105.45 83.82) (width 0.2) (layer "F.Cu") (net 16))
 (segment (start 103.9175 86.849) (end 104.95 85.8165) (width 0.2) (layer "F.Cu") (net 15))
 (segment (start 104.95 85.8165) (end 104.95 83.82) (width 0.2) (layer "F.Cu") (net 15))
 (segment (start 102.98 86.849) (end 103.9175 86.849) (width 0.2) (layer "F.Cu") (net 15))
 (segment (start 96.544 94.996) (end 98.568 94.996) (width 0.2) (layer "F.Cu") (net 9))
 (segment (start 108.856 88.799) (end 107.9185 88.799) (width 0.2) (layer "F.Cu") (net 28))
 (segment (start 106.95 87.8305) (end 106.95 83.82) (width 0.2) (layer "F.Cu") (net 28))
 (segment (start 113.1925 92.5475) (end 113.284 92.456) (width 0.2) (layer "F.Cu") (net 28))
 (segment (start 107.9185 88.799) (end 106.95 87.8305) (width 0.2) (layer "F.Cu") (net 28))
 (segment (start 103.124 79.756) (end 103.124 79.732) (width 0.2) (layer "F.Cu") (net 30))
 (segment (start 96.544 97.536) (end 98.568 97.536) (width 0.2) (layer "F.Cu") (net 22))
 (segment (start 103.9175 88.149) (end 105.95 86.1165) (width 0.2) (layer "F.Cu") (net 17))
 (segment (start 106.172 102.078) (end 106.202 102.108) (width 0.2) (layer "F.Cu") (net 17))
 (segment (start 102.98 88.149) (end 103.9175 88.149) (width 0.2) (layer "F.Cu") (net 17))
 (segment (start 105.95 86.1165) (end 105.95 83.82) (width 0.2) (layer "F.Cu") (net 17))
 (segment (start 113.03 102.616) (end 113.284 102.616) (width 0.2) (layer "F.Cu") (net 2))
 (segment (start 104.45 85.697) (end 104.45 83.82) (width 0.2) (layer "F.Cu") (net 14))
 (segment (start 102.98 86.199) (end 103.948 86.199) (width 0.2) (layer "F.Cu") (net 14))
 (segment (start 103.948 86.199) (end 104.45 85.697) (width 0.2) (layer "F.Cu") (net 14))
 (segment (start 103.910092 88.799) (end 106.45 86.259092) (width 0.2) (layer "F.Cu") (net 18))
 (segment (start 106.45 86.259092) (end 106.45 83.82) (width 0.2) (layer "F.Cu") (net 18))
 (segment (start 102.98 88.799) (end 103.910092 88.799) (width 0.2) (layer "F.Cu") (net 18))
 (segment (start 96.528 87.376) (end 98.552 87.376) (width 0.2) (layer "F.Cu") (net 21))
 (segment (start 96.544 100.076) (end 98.568 100.076) (width 0.2) (layer "F.Cu") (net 12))
 (segment (start 98.02 102.616) (end 98.171 102.616) (width 0.2) (layer "F.Cu") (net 23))
 (segment (start 98.552 79.756) (end 98.02 79.756) (width 0.2) (layer "F.Cu") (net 1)))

